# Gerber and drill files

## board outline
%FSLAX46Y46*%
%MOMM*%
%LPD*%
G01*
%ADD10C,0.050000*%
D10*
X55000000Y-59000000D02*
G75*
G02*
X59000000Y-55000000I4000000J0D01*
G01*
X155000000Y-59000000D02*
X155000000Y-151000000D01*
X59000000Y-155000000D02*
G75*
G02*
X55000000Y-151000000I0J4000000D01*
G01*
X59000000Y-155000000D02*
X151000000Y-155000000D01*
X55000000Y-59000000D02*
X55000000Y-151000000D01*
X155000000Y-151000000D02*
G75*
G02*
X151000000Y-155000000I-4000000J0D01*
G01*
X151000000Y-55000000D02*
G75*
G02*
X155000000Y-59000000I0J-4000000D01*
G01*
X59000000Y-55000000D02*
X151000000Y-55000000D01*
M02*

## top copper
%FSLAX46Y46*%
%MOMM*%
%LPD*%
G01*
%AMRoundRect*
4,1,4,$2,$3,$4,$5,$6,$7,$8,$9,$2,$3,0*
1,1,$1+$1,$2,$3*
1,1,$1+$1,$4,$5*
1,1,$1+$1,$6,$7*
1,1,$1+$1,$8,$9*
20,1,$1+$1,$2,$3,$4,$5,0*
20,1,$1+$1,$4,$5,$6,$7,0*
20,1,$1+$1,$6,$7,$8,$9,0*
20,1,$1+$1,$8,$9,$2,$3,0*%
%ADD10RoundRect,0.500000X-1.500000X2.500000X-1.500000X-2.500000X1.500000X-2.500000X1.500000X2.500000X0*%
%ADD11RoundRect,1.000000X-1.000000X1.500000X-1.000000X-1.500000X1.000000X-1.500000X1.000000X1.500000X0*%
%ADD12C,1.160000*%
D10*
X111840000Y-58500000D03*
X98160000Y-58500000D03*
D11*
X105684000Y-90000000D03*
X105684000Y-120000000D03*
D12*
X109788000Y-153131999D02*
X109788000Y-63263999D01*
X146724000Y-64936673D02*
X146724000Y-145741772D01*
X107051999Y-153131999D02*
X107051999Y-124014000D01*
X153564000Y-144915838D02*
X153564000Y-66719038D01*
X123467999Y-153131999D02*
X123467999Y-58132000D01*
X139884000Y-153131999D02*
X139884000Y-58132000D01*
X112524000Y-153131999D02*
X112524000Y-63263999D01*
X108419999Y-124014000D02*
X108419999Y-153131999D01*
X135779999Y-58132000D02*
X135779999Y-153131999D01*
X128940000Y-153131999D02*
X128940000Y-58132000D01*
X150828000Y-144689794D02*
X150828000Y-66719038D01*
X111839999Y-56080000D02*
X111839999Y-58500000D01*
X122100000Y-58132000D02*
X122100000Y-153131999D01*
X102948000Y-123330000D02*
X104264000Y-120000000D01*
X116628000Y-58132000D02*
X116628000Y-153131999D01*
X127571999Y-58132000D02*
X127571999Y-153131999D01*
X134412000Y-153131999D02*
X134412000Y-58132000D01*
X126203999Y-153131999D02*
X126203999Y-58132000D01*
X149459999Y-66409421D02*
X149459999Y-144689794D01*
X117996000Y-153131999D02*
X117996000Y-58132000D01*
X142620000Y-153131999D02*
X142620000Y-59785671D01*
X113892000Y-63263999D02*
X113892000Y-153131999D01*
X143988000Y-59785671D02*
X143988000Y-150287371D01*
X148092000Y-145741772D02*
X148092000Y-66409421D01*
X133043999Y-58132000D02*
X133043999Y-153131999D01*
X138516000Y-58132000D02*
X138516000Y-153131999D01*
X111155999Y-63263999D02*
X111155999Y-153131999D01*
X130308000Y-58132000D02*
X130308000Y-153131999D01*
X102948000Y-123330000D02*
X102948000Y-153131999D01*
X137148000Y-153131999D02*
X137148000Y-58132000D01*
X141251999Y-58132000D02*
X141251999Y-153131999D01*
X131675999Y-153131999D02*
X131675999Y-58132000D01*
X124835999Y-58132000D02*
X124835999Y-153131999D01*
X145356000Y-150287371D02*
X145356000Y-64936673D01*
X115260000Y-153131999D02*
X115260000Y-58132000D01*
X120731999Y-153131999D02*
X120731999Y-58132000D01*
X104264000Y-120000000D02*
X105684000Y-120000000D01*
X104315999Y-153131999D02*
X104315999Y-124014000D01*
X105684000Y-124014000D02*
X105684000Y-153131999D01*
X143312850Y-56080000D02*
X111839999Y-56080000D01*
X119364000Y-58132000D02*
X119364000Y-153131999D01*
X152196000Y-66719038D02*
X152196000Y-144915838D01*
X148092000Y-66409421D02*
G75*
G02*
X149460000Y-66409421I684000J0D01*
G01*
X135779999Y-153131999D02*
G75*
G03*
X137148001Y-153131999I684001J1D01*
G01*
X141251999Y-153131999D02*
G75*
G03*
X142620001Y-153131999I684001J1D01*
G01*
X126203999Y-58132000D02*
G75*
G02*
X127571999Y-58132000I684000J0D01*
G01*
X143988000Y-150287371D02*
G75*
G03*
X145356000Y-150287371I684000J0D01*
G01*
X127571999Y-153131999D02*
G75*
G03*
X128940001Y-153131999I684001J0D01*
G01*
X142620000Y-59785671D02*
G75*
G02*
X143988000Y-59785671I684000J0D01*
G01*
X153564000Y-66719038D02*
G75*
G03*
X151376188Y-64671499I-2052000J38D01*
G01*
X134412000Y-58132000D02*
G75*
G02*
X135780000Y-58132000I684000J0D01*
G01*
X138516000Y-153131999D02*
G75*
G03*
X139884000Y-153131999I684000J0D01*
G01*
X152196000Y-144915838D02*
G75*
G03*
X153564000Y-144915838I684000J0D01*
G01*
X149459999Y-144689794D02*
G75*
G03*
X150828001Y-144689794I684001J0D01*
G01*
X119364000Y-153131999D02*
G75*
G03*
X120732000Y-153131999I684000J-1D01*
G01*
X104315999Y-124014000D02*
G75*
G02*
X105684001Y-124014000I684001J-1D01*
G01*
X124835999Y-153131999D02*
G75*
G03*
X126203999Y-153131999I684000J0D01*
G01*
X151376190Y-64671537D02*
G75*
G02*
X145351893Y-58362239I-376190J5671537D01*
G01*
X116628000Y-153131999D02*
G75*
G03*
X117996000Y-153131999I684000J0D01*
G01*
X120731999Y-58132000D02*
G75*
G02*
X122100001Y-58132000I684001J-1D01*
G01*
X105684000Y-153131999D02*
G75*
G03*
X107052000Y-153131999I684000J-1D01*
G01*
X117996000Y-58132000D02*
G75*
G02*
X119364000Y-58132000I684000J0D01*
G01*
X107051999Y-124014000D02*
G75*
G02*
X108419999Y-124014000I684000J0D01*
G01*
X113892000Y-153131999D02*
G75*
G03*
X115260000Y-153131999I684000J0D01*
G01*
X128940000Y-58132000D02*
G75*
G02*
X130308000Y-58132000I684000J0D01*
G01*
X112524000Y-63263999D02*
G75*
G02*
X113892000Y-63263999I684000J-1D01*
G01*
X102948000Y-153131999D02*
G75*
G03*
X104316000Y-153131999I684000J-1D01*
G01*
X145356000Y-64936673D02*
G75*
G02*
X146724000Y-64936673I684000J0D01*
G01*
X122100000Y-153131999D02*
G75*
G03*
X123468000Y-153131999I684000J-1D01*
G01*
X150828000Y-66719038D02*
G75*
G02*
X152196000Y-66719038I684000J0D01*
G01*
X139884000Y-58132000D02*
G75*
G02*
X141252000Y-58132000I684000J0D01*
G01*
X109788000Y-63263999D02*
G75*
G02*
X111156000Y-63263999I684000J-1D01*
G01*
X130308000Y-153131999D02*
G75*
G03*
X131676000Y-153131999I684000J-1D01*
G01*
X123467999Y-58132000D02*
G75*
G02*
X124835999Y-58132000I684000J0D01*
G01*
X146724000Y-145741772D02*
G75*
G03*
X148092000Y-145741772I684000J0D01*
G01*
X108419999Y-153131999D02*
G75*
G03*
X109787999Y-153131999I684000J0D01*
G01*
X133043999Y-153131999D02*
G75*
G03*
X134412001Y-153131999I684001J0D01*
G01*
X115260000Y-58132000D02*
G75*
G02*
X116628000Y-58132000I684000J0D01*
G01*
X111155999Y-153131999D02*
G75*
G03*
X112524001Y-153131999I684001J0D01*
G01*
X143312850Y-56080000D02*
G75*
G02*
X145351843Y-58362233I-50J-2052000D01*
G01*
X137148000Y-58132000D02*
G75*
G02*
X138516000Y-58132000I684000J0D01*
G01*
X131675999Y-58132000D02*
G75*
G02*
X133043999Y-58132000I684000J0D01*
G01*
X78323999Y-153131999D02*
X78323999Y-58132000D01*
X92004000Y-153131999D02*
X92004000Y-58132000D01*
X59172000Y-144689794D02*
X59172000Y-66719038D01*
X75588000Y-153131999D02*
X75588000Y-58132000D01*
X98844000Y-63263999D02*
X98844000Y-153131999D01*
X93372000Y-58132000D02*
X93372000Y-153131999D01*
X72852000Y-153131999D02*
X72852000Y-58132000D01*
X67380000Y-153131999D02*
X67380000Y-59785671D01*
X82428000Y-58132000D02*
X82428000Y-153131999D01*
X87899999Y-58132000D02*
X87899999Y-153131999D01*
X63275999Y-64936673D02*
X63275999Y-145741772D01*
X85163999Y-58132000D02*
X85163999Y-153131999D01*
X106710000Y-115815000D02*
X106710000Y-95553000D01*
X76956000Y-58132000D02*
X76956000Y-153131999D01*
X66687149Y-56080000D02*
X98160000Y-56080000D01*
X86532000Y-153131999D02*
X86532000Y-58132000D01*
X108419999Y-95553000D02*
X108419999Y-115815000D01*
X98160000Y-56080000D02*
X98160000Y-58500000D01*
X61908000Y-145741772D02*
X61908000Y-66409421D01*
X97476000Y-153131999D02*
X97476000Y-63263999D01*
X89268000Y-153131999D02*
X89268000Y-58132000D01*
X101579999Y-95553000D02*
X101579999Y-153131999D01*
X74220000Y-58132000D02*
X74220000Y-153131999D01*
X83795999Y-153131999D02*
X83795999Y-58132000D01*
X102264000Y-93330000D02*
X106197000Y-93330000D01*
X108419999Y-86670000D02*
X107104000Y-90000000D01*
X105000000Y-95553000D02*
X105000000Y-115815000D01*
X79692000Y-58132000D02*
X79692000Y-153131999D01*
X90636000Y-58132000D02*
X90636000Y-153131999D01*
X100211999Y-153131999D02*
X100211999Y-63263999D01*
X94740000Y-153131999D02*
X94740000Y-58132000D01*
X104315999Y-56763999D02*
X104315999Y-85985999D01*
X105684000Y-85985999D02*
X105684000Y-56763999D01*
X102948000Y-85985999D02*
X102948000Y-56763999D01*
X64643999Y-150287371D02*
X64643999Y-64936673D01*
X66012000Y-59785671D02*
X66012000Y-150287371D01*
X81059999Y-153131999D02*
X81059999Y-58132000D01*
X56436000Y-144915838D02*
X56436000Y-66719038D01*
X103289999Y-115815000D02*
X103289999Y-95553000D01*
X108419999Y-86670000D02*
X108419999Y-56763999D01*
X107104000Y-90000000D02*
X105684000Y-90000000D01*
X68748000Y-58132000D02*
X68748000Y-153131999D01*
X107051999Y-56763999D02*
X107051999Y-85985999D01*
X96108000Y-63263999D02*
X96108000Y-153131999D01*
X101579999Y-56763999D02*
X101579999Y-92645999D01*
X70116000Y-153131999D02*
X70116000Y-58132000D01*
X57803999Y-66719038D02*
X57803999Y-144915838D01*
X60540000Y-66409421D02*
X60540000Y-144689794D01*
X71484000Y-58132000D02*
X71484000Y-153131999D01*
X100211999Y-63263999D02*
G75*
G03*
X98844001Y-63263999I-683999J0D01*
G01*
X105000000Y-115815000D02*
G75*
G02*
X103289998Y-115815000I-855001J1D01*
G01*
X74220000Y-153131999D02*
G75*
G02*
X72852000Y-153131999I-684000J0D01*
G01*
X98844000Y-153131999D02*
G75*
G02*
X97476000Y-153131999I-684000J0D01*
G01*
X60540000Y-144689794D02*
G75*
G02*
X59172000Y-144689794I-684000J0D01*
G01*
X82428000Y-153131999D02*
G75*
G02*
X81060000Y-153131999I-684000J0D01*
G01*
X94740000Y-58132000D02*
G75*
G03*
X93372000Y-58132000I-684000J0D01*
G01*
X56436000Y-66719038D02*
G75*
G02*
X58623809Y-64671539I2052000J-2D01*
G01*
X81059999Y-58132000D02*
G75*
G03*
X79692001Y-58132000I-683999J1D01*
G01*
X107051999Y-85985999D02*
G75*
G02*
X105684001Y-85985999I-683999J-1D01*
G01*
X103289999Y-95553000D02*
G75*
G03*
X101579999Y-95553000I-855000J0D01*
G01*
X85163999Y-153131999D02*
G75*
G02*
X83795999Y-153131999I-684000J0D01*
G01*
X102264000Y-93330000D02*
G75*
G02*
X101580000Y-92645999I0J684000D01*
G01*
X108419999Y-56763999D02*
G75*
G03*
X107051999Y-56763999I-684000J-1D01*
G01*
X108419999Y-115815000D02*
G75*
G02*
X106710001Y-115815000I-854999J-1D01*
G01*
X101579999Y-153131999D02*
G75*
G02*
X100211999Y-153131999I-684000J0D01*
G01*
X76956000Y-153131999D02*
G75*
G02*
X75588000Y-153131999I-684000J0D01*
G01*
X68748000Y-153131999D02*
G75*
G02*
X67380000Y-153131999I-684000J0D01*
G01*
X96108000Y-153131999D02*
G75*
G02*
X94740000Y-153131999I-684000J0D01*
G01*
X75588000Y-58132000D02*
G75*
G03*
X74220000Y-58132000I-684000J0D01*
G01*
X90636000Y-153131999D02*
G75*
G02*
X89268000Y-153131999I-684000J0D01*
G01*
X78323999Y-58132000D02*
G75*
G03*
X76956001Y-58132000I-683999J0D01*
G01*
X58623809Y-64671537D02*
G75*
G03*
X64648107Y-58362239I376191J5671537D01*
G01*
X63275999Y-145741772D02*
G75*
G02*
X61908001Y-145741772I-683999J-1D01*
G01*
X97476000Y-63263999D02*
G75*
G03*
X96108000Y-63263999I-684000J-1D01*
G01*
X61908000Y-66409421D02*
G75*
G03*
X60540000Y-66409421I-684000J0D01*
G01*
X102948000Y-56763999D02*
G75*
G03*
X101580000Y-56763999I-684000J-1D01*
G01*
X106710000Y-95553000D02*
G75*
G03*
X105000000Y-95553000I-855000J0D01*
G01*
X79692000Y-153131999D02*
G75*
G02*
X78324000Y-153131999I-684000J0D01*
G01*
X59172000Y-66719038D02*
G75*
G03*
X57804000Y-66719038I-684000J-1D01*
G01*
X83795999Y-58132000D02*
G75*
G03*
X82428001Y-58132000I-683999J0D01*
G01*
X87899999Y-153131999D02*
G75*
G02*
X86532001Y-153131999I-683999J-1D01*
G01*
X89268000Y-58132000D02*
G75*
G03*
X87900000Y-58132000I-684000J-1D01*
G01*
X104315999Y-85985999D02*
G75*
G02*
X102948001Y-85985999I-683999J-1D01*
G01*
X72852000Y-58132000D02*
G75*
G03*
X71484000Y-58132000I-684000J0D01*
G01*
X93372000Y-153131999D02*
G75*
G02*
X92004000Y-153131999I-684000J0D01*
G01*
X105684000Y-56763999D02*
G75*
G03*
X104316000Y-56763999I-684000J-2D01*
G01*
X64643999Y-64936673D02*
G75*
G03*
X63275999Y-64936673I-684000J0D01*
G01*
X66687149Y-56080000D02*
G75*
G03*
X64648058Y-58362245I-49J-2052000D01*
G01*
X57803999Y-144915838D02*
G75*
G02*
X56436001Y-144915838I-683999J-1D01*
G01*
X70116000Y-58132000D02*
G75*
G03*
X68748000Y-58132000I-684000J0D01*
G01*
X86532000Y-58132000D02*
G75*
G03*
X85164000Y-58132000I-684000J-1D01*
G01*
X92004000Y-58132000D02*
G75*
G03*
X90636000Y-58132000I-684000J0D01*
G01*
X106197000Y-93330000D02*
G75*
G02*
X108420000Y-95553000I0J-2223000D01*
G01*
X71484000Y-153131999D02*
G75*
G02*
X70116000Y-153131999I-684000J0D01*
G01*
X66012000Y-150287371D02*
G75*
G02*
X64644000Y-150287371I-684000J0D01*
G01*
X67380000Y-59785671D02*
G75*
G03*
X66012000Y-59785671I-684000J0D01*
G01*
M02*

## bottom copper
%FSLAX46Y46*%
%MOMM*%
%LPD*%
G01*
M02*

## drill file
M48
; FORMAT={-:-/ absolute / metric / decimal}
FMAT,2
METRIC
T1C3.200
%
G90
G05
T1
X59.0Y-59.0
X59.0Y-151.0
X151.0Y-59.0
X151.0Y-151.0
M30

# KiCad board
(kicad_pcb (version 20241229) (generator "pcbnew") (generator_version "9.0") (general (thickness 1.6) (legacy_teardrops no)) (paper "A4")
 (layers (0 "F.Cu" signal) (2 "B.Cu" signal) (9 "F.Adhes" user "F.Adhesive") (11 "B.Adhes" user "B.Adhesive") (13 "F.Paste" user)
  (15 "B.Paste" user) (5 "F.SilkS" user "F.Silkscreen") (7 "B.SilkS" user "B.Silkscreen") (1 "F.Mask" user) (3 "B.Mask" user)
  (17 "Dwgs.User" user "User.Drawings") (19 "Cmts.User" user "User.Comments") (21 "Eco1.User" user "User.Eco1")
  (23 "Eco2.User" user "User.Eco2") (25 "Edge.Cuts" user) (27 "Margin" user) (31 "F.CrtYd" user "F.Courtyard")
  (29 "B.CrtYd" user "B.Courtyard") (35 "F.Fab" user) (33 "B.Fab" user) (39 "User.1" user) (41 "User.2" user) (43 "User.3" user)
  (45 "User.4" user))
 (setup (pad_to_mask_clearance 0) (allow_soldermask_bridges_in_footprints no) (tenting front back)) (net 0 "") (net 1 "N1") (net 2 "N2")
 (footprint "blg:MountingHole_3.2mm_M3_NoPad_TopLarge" (layer "F.Cu") (at 151 59)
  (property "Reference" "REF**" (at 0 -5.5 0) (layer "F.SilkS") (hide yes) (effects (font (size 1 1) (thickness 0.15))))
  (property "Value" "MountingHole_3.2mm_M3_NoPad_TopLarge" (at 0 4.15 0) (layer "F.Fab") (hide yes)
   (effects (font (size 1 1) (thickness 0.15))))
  (pad "" np_thru_hole circle (at 0 0) (size 7.6 7.6) (drill 3.2) (layers) (zone_connect 2)))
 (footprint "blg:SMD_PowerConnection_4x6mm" (layer "F.Cu") (at 111.84 58.5 -90)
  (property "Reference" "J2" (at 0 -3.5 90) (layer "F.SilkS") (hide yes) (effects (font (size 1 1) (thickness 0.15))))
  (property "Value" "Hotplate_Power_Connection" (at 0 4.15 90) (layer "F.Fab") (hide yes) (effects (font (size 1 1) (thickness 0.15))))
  (pad "1" smd roundrect (at 0 0 270) (size 6 4) (layers "F.Cu" "F.Mask" "F.Paste") (roundrect_rratio 0.125) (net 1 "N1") (zone_connect 2)))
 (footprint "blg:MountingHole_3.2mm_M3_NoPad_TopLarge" (layer "F.Cu") (at 59 151)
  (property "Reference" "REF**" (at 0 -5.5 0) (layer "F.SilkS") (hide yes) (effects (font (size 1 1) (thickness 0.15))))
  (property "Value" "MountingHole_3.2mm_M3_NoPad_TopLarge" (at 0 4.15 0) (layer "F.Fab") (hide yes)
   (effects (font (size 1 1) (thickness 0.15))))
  (pad "" np_thru_hole circle (at 0 0) (size 7.6 7.6) (drill 3.2) (layers) (zone_connect 2)))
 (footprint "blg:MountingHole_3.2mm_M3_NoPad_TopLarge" (layer "F.Cu") (at 151 151)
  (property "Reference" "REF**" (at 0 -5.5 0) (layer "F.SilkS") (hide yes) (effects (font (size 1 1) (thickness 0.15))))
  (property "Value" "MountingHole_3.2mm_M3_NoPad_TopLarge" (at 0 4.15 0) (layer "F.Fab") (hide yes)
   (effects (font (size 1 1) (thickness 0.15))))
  (pad "" np_thru_hole circle (at 0 0) (size 7.6 7.6) (drill 3.2) (layers) (zone_connect 2)))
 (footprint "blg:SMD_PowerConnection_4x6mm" (layer "F.Cu") (at 98.16 58.5 -90)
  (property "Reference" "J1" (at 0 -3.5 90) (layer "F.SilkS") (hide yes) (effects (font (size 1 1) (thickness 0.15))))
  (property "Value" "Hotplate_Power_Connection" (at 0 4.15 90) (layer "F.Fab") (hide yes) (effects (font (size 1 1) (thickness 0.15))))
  (pad "1" smd roundrect (at 0 0 270) (size 6 4) (layers "F.Cu" "F.Mask" "F.Paste") (roundrect_rratio 0.125) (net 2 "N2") (zone_connect 2)))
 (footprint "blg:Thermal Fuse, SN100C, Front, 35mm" (layer "F.Cu") (at 105.684 105 -90)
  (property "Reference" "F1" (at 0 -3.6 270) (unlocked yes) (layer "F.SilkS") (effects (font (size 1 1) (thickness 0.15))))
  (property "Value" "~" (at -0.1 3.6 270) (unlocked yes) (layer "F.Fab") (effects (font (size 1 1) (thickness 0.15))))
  (pad "1" smd roundrect (at -15 0 270) (size 5 4) (layers "F.Cu" "F.Mask") (roundrect_rratio 0.25) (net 2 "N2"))
  (pad "2" smd roundrect (at 15 0 270) (size 5 4) (layers "F.Cu" "F.Mask") (roundrect_rratio 0.25) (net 1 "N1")))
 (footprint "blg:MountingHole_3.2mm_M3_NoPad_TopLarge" (layer "F.Cu") (at 59 59)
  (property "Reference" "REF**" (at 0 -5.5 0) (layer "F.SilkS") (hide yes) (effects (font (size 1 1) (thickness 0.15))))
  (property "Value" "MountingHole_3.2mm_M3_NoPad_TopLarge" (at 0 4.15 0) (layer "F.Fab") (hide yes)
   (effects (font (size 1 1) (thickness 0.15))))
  (pad "" np_thru_hole circle (at 0 0) (size 7.6 7.6) (drill 3.2) (layers) (zone_connect 2)))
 (gr_arc (start 55 59) (mid 56.171573 56.171573) (end 59 55) (stroke (width 0.05) (type solid)) (layer "Edge.Cuts"))
 (gr_line (start 155 59) (end 155 151) (stroke (width 0.05) (type default)) (layer "Edge.Cuts"))
 (gr_arc (start 59 155) (mid 56.171573 153.828427) (end 55 151) (stroke (width 0.05) (type solid)) (layer "Edge.Cuts"))
 (gr_line (start 59 155) (end 151 155) (stroke (width 0.05) (type default)) (layer "Edge.Cuts"))
 (gr_line (start 55 59) (end 55 151) (stroke (width 0.05) (type default)) (layer "Edge.Cuts"))
 (gr_arc (start 155 151) (mid 153.828427 153.828427) (end 151 155) (stroke (width 0.05) (type solid)) (layer "Edge.Cuts"))
 (gr_arc (start 151 55) (mid 153.828427 56.171573) (end 155 59) (stroke (width 0.05) (type solid)) (layer "Edge.Cuts"))
 (gr_line (start 59 55) (end 151 55) (stroke (width 0.05) (type default)) (layer "Edge.Cuts"))
 (segment (start 109.788 153.131999) (end 109.788 63.263999) (width 1.16) (layer "F.Cu") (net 1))
 (segment (start 146.724 64.936673) (end 146.724 145.741772) (width 1.16) (layer "F.Cu") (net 1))
 (segment (start 107.051999 153.131999) (end 107.051999 124.014) (width 1.16) (layer "F.Cu") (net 1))
 (segment (start 153.564 144.915838) (end 153.564 66.719038) (width 1.16) (layer "F.Cu") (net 1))
 (segment (start 123.467999 153.131999) (end 123.467999 58.132) (width 1.16) (layer "F.Cu") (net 1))
 (segment (start 139.884 153.131999) (end 139.884 58.132) (width 1.16) (layer "F.Cu") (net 1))
 (segment (start 112.524 153.131999) (end 112.524 63.263999) (width 1.16) (layer "F.Cu") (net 1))
 (segment (start 108.419999 124.014) (end 108.419999 153.131999) (width 1.16) (layer "F.Cu") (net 1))
 (segment (start 135.779999 58.132) (end 135.779999 153.131999) (width 1.16) (layer "F.Cu") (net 1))
 (segment (start 128.94 153.131999) (end 128.94 58.132) (width 1.16) (layer "F.Cu") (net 1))
 (segment (start 150.828 144.689794) (end 150.828 66.719038) (width 1.16) (layer "F.Cu") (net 1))
 (segment (start 111.839999 56.08) (end 111.839999 58.5) (width 1.16) (layer "F.Cu") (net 1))
 (segment (start 122.1 58.132) (end 122.1 153.131999) (width 1.16) (layer "F.Cu") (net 1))
 (segment (start 102.948 123.33) (end 104.264 120) (width 1.16) (layer "F.Cu") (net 1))
 (segment (start 116.628 58.132) (end 116.628 153.131999) (width 1.16) (layer "F.Cu") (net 1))
 (segment (start 127.571999 58.132) (end 127.571999 153.131999) (width 1.16) (layer "F.Cu") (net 1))
 (segment (start 134.412 153.131999) (end 134.412 58.132) (width 1.16) (layer "F.Cu") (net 1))
 (segment (start 126.203999 153.131999) (end 126.203999 58.132) (width 1.16) (layer "F.Cu") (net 1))
 (segment (start 149.459999 66.409421) (end 149.459999 144.689794) (width 1.16) (layer "F.Cu") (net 1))
 (segment (start 117.996 153.131999) (end 117.996 58.132) (width 1.16) (layer "F.Cu") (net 1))
 (segment (start 142.62 153.131999) (end 142.62 59.785671) (width 1.16) (layer "F.Cu") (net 1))
 (segment (start 113.892 63.263999) (end 113.892 153.131999) (width 1.16) (layer "F.Cu") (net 1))
 (segment (start 143.988 59.785671) (end 143.988 150.287371) (width 1.16) (layer "F.Cu") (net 1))
 (segment (start 148.092 145.741772) (end 148.092 66.409421) (width 1.16) (layer "F.Cu") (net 1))
 (segment (start 133.043999 58.132) (end 133.043999 153.131999) (width 1.16) (layer "F.Cu") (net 1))
 (segment (start 138.516 58.132) (end 138.516 153.131999) (width 1.16) (layer "F.Cu") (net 1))
 (segment (start 111.155999 63.263999) (end 111.155999 153.131999) (width 1.16) (layer "F.Cu") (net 1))
 (segment (start 130.308 58.132) (end 130.308 153.131999) (width 1.16) (layer "F.Cu") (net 1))
 (segment (start 102.948 123.33) (end 102.948 153.131999) (width 1.16) (layer "F.Cu") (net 1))
 (segment (start 137.148 153.131999) (end 137.148 58.132) (width 1.16) (layer "F.Cu") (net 1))
 (segment (start 141.251999 58.132) (end 141.251999 153.131999) (width 1.16) (layer "F.Cu") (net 1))
 (segment (start 131.675999 153.131999) (end 131.675999 58.132) (width 1.16) (layer "F.Cu") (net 1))
 (segment (start 124.835999 58.132) (end 124.835999 153.131999) (width 1.16) (layer "F.Cu") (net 1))
 (segment (start 145.356 150.287371) (end 145.356 64.936673) (width 1.16) (layer "F.Cu") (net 1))
 (segment (start 115.26 153.131999) (end 115.26 58.132) (width 1.16) (layer "F.Cu") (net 1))
 (segment (start 120.731999 153.131999) (end 120.731999 58.132) (width 1.16) (layer "F.Cu") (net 1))
 (segment (start 104.264 120) (end 105.684 120) (width 1.16) (layer "F.Cu") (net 1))
 (segment (start 104.315999 153.131999) (end 104.315999 124.014) (width 1.16) (layer "F.Cu") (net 1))
 (segment (start 105.684 124.014) (end 105.684 153.131999) (width 1.16) (layer "F.Cu") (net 1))
 (segment (start 143.31285 56.08) (end 111.839999 56.08) (width 1.16) (layer "F.Cu") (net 1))
 (segment (start 119.364 58.132) (end 119.364 153.131999) (width 1.16) (layer "F.Cu") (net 1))
 (segment (start 152.196 66.719038) (end 152.196 144.915838) (width 1.16) (layer "F.Cu") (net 1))
 (arc (start 148.092 66.409421) (mid 148.775999 65.725421) (end 149.459999 66.409421) (width 1.16) (layer "F.Cu") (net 1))
 (arc (start 135.779999 153.131999) (mid 136.464 153.815999) (end 137.148 153.131999) (width 1.16) (layer "F.Cu") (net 1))
 (arc (start 141.251999 153.131999) (mid 141.936 153.815999) (end 142.62 153.131999) (width 1.16) (layer "F.Cu") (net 1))
 (arc (start 126.203999 58.132) (mid 126.888 57.448) (end 127.571999 58.132) (width 1.16) (layer "F.Cu") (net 1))
 (arc (start 143.988 150.287371) (mid 144.672 150.971371) (end 145.356 150.287371) (width 1.16) (layer "F.Cu") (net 1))
 (arc (start 127.571999 153.131999) (mid 128.255999 153.815999) (end 128.94 153.131999) (width 1.16) (layer "F.Cu") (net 1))
 (arc (start 142.62 59.785671) (mid 143.303999 59.101671) (end 143.988 59.785671) (width 1.16) (layer "F.Cu") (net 1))
 (arc (start 153.564 66.719038) (mid 153.008247 65.314778) (end 151.37619 64.671537) (width 1.16) (layer "F.Cu") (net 1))
 (arc (start 134.412 58.132) (mid 135.096 57.448) (end 135.779999 58.132) (width 1.16) (layer "F.Cu") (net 1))
 (arc (start 138.516 153.131999) (mid 139.2 153.815999) (end 139.884 153.131999) (width 1.16) (layer "F.Cu") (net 1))
 (arc (start 152.196 144.915838) (mid 152.88 145.599838) (end 153.564 144.915838) (width 1.16) (layer "F.Cu") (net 1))
 (arc (start 149.459999 144.689794) (mid 150.144 145.373794) (end 150.828 144.689794) (width 1.16) (layer "F.Cu") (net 1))
 (arc (start 119.364 153.131999) (mid 120.047999 153.815999) (end 120.731999 153.131999) (width 1.16) (layer "F.Cu") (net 1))
 (arc (start 104.315999 124.014) (mid 105 123.33) (end 105.684 124.014) (width 1.16) (layer "F.Cu") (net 1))
 (arc (start 124.835999 153.131999) (mid 125.52 153.815999) (end 126.203999 153.131999) (width 1.16) (layer "F.Cu") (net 1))
 (arc (start 151.37619 64.671537) (mid 146.889028 62.925273) (end 145.351892 58.362239) (width 1.16) (layer "F.Cu") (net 1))
 (arc (start 116.628 153.131999) (mid 117.312 153.815999) (end 117.996 153.131999) (width 1.16) (layer "F.Cu") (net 1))
 (arc (start 120.731999 58.132) (mid 121.416 57.448) (end 122.1 58.132) (width 1.16) (layer "F.Cu") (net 1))
 (arc (start 105.684 153.131999) (mid 106.368 153.815999) (end 107.051999 153.131999) (width 1.16) (layer "F.Cu") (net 1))
 (arc (start 117.996 58.132) (mid 118.68 57.448) (end 119.364 58.132) (width 1.16) (layer "F.Cu") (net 1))
 (arc (start 107.051999 124.014) (mid 107.736 123.33) (end 108.419999 124.014) (width 1.16) (layer "F.Cu") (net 1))
 (arc (start 113.892 153.131999) (mid 114.576 153.815999) (end 115.26 153.131999) (width 1.16) (layer "F.Cu") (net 1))
 (arc (start 128.94 58.132) (mid 129.624 57.448) (end 130.308 58.132) (width 1.16) (layer "F.Cu") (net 1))
 (arc (start 112.524 63.263999) (mid 113.207999 62.58) (end 113.892 63.263999) (width 1.16) (layer "F.Cu") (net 1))
 (arc (start 102.948 153.131999) (mid 103.632 153.815999) (end 104.315999 153.131999) (width 1.16) (layer "F.Cu") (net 1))
 (arc (start 145.356 64.936673) (mid 146.04 64.252673) (end 146.724 64.936673) (width 1.16) (layer "F.Cu") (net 1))
 (arc (start 122.1 153.131999) (mid 122.783999 153.815999) (end 123.467999 153.131999) (width 1.16) (layer "F.Cu") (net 1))
 (arc (start 150.828 66.719038) (mid 151.511999 66.035038) (end 152.196 66.719038) (width 1.16) (layer "F.Cu") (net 1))
 (arc (start 139.884 58.132) (mid 140.568 57.448) (end 141.251999 58.132) (width 1.16) (layer "F.Cu") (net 1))
 (arc (start 109.788 63.263999) (mid 110.472 62.58) (end 111.155999 63.263999) (width 1.16) (layer "F.Cu") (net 1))
 (arc (start 130.308 153.131999) (mid 130.991999 153.815999) (end 131.675999 153.131999) (width 1.16) (layer "F.Cu") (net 1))
 (arc (start 123.467999 58.132) (mid 124.152 57.448) (end 124.835999 58.132) (width 1.16) (layer "F.Cu") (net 1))
 (arc (start 146.724 145.741772) (mid 147.408 146.425772) (end 148.092 145.741772) (width 1.16) (layer "F.Cu") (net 1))
 (arc (start 108.419999 153.131999) (mid 109.104 153.815999) (end 109.787999 153.131999) (width 1.16) (layer "F.Cu") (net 1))
 (arc (start 133.043999 153.131999) (mid 133.727999 153.815999) (end 134.412 153.131999) (width 1.16) (layer "F.Cu") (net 1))
 (arc (start 115.26 58.132) (mid 115.943999 57.448) (end 116.628 58.132) (width 1.16) (layer "F.Cu") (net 1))
 (arc (start 111.155999 153.131999) (mid 111.839999 153.815999) (end 112.524 153.131999) (width 1.16) (layer "F.Cu") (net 1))
 (arc (start 143.31285 56.08) (mid 144.843071 56.76484) (end 145.351892 58.362239) (width 1.16) (layer "F.Cu") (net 1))
 (arc (start 137.148 58.132) (mid 137.832 57.448) (end 138.516 58.132) (width 1.16) (layer "F.Cu") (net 1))
 (arc (start 131.675999 58.132) (mid 132.36 57.448) (end 133.043999 58.132) (width 1.16) (layer "F.Cu") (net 1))
 (segment (start 78.323999 153.131999) (end 78.323999 58.132) (width 1.16) (layer "F.Cu") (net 2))
 (segment (start 92.004 153.131999) (end 92.004 58.132) (width 1.16) (layer "F.Cu") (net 2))
 (segment (start 59.172 144.689794) (end 59.172 66.719038) (width 1.16) (layer "F.Cu") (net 2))
 (segment (start 75.588 153.131999) (end 75.588 58.132) (width 1.16) (layer "F.Cu") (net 2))
 (segment (start 98.844 63.263999) (end 98.844 153.131999) (width 1.16) (layer "F.Cu") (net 2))
 (segment (start 93.372 58.132) (end 93.372 153.131999) (width 1.16) (layer "F.Cu") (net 2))
 (segment (start 72.852 153.131999) (end 72.852 58.132) (width 1.16) (layer "F.Cu") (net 2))
 (segment (start 67.38 153.131999) (end 67.38 59.785671) (width 1.16) (layer "F.Cu") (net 2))
 (segment (start 82.428 58.132) (end 82.428 153.131999) (width 1.16) (layer "F.Cu") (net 2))
 (segment (start 87.899999 58.132) (end 87.899999 153.131999) (width 1.16) (layer "F.Cu") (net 2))
 (segment (start 63.275999 64.936673) (end 63.275999 145.741772) (width 1.16) (layer "F.Cu") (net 2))
 (segment (start 85.163999 58.132) (end 85.163999 153.131999) (width 1.16) (layer "F.Cu") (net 2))
 (segment (start 106.71 115.815) (end 106.71 95.553) (width 1.16) (layer "F.Cu") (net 2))
 (segment (start 76.956 58.132) (end 76.956 153.131999) (width 1.16) (layer "F.Cu") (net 2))
 (segment (start 66.687149 56.08) (end 98.16 56.08) (width 1.16) (layer "F.Cu") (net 2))
 (segment (start 86.532 153.131999) (end 86.532 58.132) (width 1.16) (layer "F.Cu") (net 2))
 (segment (start 108.419999 95.553) (end 108.419999 115.815) (width 1.16) (layer "F.Cu") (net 2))
 (segment (start 98.16 56.08) (end 98.16 58.5) (width 1.16) (layer "F.Cu") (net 2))
 (segment (start 61.908 145.741772) (end 61.908 66.409421) (width 1.16) (layer "F.Cu") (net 2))
 (segment (start 97.476 153.131999) (end 97.476 63.263999) (width 1.16) (layer "F.Cu") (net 2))
 (segment (start 89.268 153.131999) (end 89.268 58.132) (width 1.16) (layer "F.Cu") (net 2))
 (segment (start 101.579999 95.553) (end 101.579999 153.131999) (width 1.16) (layer "F.Cu") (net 2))
 (segment (start 74.22 58.132) (end 74.22 153.131999) (width 1.16) (layer "F.Cu") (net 2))
 (segment (start 83.795999 153.131999) (end 83.795999 58.132) (width 1.16) (layer "F.Cu") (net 2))
 (segment (start 102.264 93.33) (end 106.197 93.33) (width 1.16) (layer "F.Cu") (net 2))
 (segment (start 108.419999 86.67) (end 107.104 90) (width 1.16) (layer "F.Cu") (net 2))
 (segment (start 105 95.553) (end 105 115.815) (width 1.16) (layer "F.Cu") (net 2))
 (segment (start 79.692 58.132) (end 79.692 153.131999) (width 1.16) (layer "F.Cu") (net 2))
 (segment (start 90.636 58.132) (end 90.636 153.131999) (width 1.16) (layer "F.Cu") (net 2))
 (segment (start 100.211999 153.131999) (end 100.211999 63.263999) (width 1.16) (layer "F.Cu") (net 2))
 (segment (start 94.74 153.131999) (end 94.74 58.132) (width 1.16) (layer "F.Cu") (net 2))
 (segment (start 104.315999 56.763999) (end 104.315999 85.985999) (width 1.16) (layer "F.Cu") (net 2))
 (segment (start 105.684 85.985999) (end 105.684 56.763999) (width 1.16) (layer "F.Cu") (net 2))
 (segment (start 102.948 85.985999) (end 102.948 56.763999) (width 1.16) (layer "F.Cu") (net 2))
 (segment (start 64.643999 150.287371) (end 64.643999 64.936673) (width 1.16) (layer "F.Cu") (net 2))
 (segment (start 66.012 59.785671) (end 66.012 150.287371) (width 1.16) (layer "F.Cu") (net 2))
 (segment (start 81.059999 153.131999) (end 81.059999 58.132) (width 1.16) (layer "F.Cu") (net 2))
 (segment (start 56.436 144.915838) (end 56.436 66.719038) (width 1.16) (layer "F.Cu") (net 2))
 (segment (start 103.289999 115.815) (end 103.289999 95.553) (width 1.16) (layer "F.Cu") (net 2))
 (segment (start 108.419999 86.67) (end 108.419999 56.763999) (width 1.16) (layer "F.Cu") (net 2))
 (segment (start 107.104 90) (end 105.684 90) (width 1.16) (layer "F.Cu") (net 2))
 (segment (start 68.748 58.132) (end 68.748 153.131999) (width 1.16) (layer "F.Cu") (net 2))
 (segment (start 107.051999 56.763999) (end 107.051999 85.985999) (width 1.16) (layer "F.Cu") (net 2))
 (segment (start 96.108 63.263999) (end 96.108 153.131999) (width 1.16) (layer "F.Cu") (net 2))
 (segment (start 101.579999 56.763999) (end 101.579999 92.645999) (width 1.16) (layer "F.Cu") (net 2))
 (segment (start 70.116 153.131999) (end 70.116 58.132) (width 1.16) (layer "F.Cu") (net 2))
 (segment (start 57.803999 66.719038) (end 57.803999 144.915838) (width 1.16) (layer "F.Cu") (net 2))
 (segment (start 60.54 66.409421) (end 60.54 144.689794) (width 1.16) (layer "F.Cu") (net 2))
 (segment (start 71.484 58.132) (end 71.484 153.131999) (width 1.16) (layer "F.Cu") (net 2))
 (arc (start 100.211999 63.263999) (mid 99.527999 62.58) (end 98.844 63.263999) (width 1.16) (layer "F.Cu") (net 2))
 (arc (start 105 115.815) (mid 104.145 116.67) (end 103.289999 115.815) (width 1.16) (layer "F.Cu") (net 2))
 (arc (start 74.22 153.131999) (mid 73.535999 153.815999) (end 72.852 153.131999) (width 1.16) (layer "F.Cu") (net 2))
 (arc (start 98.844 153.131999) (mid 98.16 153.815999) (end 97.476 153.131999) (width 1.16) (layer "F.Cu") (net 2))
 (arc (start 60.54 144.689794) (mid 59.856 145.373794) (end 59.172 144.689794) (width 1.16) (layer "F.Cu") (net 2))
 (arc (start 82.428 153.131999) (mid 81.744 153.815999) (end 81.059999 153.131999) (width 1.16) (layer "F.Cu") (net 2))
 (arc (start 94.74 58.132) (mid 94.056 57.448) (end 93.372 58.132) (width 1.16) (layer "F.Cu") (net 2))
 (arc (start 56.436 66.719038) (mid 56.991752 65.314778) (end 58.623809 64.671537) (width 1.16) (layer "F.Cu") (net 2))
 (arc (start 81.059999 58.132) (mid 80.376 57.448) (end 79.692 58.132) (width 1.16) (layer "F.Cu") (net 2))
 (arc (start 107.051999 85.985999) (mid 106.368 86.67) (end 105.684 85.985999) (width 1.16) (layer "F.Cu") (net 2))
 (arc (start 103.289999 95.553) (mid 102.435 94.698) (end 101.579999 95.553) (width 1.16) (layer "F.Cu") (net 2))
 (arc (start 85.163999 153.131999) (mid 84.48 153.815999) (end 83.795999 153.131999) (width 1.16) (layer "F.Cu") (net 2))
 (arc (start 102.264 93.33) (mid 101.780338 93.129661) (end 101.579999 92.645999) (width 1.16) (layer "F.Cu") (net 2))
 (arc (start 108.419999 56.763999) (mid 107.736 56.08) (end 107.051999 56.763999) (width 1.16) (layer "F.Cu") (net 2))
 (arc (start 108.419999 115.815) (mid 107.565 116.67) (end 106.71 115.815) (width 1.16) (layer "F.Cu") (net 2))
 (arc (start 101.579999 153.131999) (mid 100.896 153.815999) (end 100.211999 153.131999) (width 1.16) (layer "F.Cu") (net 2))
 (arc (start 76.956 153.131999) (mid 76.271999 153.815999) (end 75.588 153.131999) (width 1.16) (layer "F.Cu") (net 2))
 (arc (start 68.748 153.131999) (mid 68.064 153.815999) (end 67.38 153.131999) (width 1.16) (layer "F.Cu") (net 2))
 (arc (start 96.108 153.131999) (mid 95.423999 153.815999) (end 94.74 153.131999) (width 1.16) (layer "F.Cu") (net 2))
 (arc (start 75.588 58.132) (mid 74.904 57.448) (end 74.22 58.132) (width 1.16) (layer "F.Cu") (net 2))
 (arc (start 90.636 153.131999) (mid 89.951999 153.815999) (end 89.268 153.131999) (width 1.16) (layer "F.Cu") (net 2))
 (arc (start 78.323999 58.132) (mid 77.64 57.448) (end 76.956 58.132) (width 1.16) (layer "F.Cu") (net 2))
 (arc (start 58.623809 64.671537) (mid 63.110971 62.925273) (end 64.648107 58.362239) (width 1.16) (layer "F.Cu") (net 2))
 (arc (start 63.275999 145.741772) (mid 62.591999 146.425772) (end 61.908 145.741772) (width 1.16) (layer "F.Cu") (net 2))
 (arc (start 97.476 63.263999) (mid 96.791999 62.58) (end 96.108 63.263999) (width 1.16) (layer "F.Cu") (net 2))
 (arc (start 61.908 66.409421) (mid 61.224 65.725421) (end 60.54 66.409421) (width 1.16) (layer "F.Cu") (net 2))
 (arc (start 102.948 56.763999) (mid 102.264 56.08) (end 101.58 56.763999) (width 1.16) (layer "F.Cu") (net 2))
 (arc (start 106.71 95.553) (mid 105.854999 94.698) (end 105 95.553) (width 1.16) (layer "F.Cu") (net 2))
 (arc (start 79.692 153.131999) (mid 79.008 153.815999) (end 78.323999 153.131999) (width 1.16) (layer "F.Cu") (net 2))
 (arc (start 59.172 66.719038) (mid 58.488 66.035038) (end 57.803999 66.719038) (width 1.16) (layer "F.Cu") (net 2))
 (arc (start 83.795999 58.132) (mid 83.112 57.448) (end 82.428 58.132) (width 1.16) (layer "F.Cu") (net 2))
 (arc (start 87.899999 153.131999) (mid 87.216 153.815999) (end 86.532 153.131999) (width 1.16) (layer "F.Cu") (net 2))
 (arc (start 89.268 58.132) (mid 88.584 57.448) (end 87.899999 58.132) (width 1.16) (layer "F.Cu") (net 2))
 (arc (start 104.315999 85.985999) (mid 103.632 86.67) (end 102.948 85.985999) (width 1.16) (layer "F.Cu") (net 2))
 (arc (start 72.852 58.132) (mid 72.167999 57.448) (end 71.484 58.132) (width 1.16) (layer "F.Cu") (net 2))
 (arc (start 93.372 153.131999) (mid 92.687999 153.815999) (end 92.004 153.131999) (width 1.16) (layer "F.Cu") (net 2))
 (arc (start 105.684 56.763999) (mid 105 56.08) (end 104.315999 56.763999) (width 1.16) (layer "F.Cu") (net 2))
 (arc (start 64.643999 64.936673) (mid 63.96 64.252673) (end 63.275999 64.936673) (width 1.16) (layer "F.Cu") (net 2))
 (arc (start 66.687149 56.08) (mid 65.156928 56.76484) (end 64.648107 58.362239) (width 1.16) (layer "F.Cu") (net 2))
 (arc (start 57.803999 144.915838) (mid 57.12 145.599838) (end 56.436 144.915838) (width 1.16) (layer "F.Cu") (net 2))
 (arc (start 70.116 58.132) (mid 69.431999 57.448) (end 68.748 58.132) (width 1.16) (layer "F.Cu") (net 2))
 (arc (start 86.532 58.132) (mid 85.848 57.448) (end 85.163999 58.132) (width 1.16) (layer "F.Cu") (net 2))
 (arc (start 92.004 58.132) (mid 91.32 57.448) (end 90.636 58.132) (width 1.16) (layer "F.Cu") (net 2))
 (arc (start 106.197 93.33) (mid 107.768898 93.981101) (end 108.419999 95.553) (width 1.16) (layer "F.Cu") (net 2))
 (arc (start 71.484 153.131999) (mid 70.8 153.815999) (end 70.116 153.131999) (width 1.16) (layer "F.Cu") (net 2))
 (arc (start 66.012 150.287371) (mid 65.328 150.971371) (end 64.643999 150.287371) (width 1.16) (layer "F.Cu") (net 2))
 (arc (start 67.38 59.785671) (mid 66.696 59.101671) (end 66.012 59.785671) (width 1.16) (layer "F.Cu") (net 2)))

